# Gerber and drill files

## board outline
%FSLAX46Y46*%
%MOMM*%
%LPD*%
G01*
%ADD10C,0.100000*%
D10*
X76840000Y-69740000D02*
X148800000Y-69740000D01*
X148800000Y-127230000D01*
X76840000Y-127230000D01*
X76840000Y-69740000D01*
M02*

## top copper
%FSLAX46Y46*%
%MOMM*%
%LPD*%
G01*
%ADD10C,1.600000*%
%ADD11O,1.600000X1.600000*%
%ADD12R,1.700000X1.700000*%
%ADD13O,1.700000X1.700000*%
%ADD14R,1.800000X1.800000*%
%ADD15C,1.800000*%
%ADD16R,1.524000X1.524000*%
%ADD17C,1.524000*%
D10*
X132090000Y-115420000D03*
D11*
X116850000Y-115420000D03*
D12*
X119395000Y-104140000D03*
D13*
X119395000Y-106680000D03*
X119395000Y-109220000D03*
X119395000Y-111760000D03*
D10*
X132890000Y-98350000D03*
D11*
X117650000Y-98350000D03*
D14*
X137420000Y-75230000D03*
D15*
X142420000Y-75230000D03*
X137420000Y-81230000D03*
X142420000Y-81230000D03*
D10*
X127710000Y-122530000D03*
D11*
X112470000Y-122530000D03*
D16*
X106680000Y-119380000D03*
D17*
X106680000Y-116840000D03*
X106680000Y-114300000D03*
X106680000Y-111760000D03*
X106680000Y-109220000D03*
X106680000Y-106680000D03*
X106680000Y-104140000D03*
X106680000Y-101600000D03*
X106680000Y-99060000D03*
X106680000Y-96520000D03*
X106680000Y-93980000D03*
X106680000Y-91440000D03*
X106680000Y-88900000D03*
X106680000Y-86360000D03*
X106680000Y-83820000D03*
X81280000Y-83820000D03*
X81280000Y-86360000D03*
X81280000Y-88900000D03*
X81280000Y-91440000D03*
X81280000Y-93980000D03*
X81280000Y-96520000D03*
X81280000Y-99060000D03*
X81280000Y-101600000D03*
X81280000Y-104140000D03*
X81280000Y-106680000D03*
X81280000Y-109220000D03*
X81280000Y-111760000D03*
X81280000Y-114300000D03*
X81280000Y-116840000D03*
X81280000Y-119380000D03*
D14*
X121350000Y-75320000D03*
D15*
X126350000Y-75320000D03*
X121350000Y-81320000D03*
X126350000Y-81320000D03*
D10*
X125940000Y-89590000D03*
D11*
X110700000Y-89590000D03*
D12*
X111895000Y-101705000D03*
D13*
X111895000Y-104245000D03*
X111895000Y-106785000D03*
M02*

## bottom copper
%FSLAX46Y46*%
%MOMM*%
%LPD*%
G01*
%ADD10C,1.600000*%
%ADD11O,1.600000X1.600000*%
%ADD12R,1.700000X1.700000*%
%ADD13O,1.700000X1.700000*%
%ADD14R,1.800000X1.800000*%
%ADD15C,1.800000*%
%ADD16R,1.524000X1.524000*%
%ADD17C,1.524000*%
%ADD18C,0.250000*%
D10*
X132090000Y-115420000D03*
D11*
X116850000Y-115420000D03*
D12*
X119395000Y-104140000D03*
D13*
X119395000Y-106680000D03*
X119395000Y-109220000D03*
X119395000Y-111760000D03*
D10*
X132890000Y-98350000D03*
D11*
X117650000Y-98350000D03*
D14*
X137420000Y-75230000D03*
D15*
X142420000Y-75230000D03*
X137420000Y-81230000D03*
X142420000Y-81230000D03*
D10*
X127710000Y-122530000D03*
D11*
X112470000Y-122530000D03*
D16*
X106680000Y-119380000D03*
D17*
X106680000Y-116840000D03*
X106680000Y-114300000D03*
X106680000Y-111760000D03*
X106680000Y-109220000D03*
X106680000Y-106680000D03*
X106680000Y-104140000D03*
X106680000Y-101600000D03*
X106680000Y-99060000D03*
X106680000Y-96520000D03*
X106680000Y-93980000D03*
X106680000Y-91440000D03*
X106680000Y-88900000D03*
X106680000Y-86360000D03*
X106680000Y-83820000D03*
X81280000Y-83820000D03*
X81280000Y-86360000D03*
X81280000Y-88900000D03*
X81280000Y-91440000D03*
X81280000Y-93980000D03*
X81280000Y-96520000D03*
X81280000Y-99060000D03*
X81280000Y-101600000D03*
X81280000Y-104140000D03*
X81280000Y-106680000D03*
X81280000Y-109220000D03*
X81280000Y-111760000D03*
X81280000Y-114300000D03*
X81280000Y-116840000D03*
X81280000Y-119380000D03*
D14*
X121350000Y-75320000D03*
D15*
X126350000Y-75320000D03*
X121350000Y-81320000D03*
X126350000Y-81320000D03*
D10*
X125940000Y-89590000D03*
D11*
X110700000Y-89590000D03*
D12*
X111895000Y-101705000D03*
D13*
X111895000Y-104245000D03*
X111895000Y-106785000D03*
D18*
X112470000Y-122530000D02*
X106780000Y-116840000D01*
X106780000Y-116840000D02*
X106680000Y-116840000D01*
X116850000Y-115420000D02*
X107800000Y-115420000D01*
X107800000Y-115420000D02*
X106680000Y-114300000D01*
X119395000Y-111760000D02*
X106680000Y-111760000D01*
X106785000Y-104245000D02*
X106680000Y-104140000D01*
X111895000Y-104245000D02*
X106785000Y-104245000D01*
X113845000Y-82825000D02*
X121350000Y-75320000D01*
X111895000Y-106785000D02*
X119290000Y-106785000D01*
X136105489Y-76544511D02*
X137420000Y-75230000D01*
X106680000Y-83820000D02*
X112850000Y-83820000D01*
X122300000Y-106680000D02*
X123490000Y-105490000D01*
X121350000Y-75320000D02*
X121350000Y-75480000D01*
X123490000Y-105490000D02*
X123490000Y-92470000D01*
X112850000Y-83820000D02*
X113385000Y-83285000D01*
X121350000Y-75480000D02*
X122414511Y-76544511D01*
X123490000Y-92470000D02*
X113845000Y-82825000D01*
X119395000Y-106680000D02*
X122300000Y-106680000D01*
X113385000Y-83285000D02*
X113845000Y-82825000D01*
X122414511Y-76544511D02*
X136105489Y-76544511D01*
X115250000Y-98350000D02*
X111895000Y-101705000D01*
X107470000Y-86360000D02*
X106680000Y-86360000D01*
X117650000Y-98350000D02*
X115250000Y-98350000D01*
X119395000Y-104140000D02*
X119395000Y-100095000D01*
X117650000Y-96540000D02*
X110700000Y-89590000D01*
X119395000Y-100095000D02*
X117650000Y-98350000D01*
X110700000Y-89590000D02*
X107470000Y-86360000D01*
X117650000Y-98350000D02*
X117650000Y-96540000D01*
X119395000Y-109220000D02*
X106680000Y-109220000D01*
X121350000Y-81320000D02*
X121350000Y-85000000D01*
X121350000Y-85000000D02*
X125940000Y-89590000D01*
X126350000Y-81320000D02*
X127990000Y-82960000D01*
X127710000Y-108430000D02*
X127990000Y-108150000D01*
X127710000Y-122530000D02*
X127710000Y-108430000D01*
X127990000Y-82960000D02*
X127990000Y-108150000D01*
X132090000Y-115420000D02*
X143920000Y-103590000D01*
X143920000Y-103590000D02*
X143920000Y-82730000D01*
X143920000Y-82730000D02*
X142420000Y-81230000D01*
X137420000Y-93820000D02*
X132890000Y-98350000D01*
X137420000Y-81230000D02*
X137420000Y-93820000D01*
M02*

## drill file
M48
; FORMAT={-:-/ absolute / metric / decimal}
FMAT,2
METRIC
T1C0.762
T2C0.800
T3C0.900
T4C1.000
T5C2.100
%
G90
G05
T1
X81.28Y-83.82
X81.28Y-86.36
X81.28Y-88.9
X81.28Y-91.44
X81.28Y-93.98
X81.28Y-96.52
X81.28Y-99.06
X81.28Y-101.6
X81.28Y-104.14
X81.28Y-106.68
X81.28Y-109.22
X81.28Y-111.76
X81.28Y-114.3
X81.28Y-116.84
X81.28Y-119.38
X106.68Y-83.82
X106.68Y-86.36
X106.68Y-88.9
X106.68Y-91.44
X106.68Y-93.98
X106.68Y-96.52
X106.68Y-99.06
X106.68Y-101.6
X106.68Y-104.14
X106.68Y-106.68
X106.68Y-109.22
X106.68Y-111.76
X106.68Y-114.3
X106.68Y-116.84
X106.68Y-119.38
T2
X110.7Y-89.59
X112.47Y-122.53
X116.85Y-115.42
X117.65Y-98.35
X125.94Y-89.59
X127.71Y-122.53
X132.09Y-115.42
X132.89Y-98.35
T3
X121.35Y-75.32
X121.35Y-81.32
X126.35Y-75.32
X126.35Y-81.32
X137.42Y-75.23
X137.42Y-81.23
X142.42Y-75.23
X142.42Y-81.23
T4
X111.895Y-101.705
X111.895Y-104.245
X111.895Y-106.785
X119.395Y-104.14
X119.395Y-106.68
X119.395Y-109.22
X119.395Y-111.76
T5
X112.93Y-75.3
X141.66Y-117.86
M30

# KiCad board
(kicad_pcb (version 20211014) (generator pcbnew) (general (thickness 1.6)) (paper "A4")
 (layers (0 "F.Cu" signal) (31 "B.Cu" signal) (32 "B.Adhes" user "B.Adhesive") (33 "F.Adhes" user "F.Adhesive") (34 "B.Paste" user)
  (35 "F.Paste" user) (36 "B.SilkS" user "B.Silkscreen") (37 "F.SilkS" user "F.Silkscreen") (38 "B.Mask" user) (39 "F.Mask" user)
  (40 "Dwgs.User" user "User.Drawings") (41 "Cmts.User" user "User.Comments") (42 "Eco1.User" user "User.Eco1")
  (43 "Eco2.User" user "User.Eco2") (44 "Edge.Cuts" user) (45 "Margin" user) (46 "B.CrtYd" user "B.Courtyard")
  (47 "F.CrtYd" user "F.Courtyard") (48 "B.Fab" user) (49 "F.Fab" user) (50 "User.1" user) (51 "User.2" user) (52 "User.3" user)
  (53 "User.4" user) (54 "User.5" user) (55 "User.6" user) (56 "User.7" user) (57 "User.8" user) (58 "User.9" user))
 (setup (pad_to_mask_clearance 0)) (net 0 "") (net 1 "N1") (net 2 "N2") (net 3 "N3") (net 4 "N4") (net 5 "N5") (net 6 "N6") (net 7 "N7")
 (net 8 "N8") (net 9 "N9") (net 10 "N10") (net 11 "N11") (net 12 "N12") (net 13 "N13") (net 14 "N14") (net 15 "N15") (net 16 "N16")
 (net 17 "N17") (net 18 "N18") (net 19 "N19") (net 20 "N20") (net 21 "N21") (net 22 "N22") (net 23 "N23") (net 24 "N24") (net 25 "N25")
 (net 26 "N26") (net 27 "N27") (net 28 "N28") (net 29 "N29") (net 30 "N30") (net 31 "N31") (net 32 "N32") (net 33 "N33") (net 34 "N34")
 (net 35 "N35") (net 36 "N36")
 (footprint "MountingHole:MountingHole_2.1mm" (layer "F.Cu") (at 112.93 75.3)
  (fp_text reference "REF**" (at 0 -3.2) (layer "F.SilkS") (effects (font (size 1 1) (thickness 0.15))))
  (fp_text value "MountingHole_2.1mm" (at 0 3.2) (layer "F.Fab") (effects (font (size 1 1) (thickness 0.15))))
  (pad "" np_thru_hole circle (at 0 0) (size 2.1 2.1) (drill 2.1) (layers *.Cu *.Mask)))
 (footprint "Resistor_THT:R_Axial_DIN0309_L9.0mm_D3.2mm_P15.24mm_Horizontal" (layer "F.Cu") (at 132.09 115.42 180)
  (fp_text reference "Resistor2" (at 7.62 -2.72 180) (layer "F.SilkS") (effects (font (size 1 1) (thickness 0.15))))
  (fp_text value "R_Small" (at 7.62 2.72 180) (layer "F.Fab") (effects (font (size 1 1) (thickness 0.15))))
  (pad "1" thru_hole circle (at 0 0 180) (size 1.6 1.6) (drill 0.8) (layers *.Cu *.Mask) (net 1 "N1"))
  (pad "2" thru_hole oval (at 15.24 0 180) (size 1.6 1.6) (drill 0.8) (layers *.Cu *.Mask) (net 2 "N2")))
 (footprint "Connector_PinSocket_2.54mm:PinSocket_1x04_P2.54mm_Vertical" (layer "F.Cu") (at 119.395 104.14)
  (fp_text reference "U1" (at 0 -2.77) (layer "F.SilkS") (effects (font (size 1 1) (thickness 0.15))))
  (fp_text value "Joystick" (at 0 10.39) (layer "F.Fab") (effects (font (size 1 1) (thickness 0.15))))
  (pad "1" thru_hole rect (at 0 0) (size 1.7 1.7) (drill 1) (layers *.Cu *.Mask) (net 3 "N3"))
  (pad "2" thru_hole oval (at 0 2.54) (size 1.7 1.7) (drill 1) (layers *.Cu *.Mask) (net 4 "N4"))
  (pad "3" thru_hole oval (at 0 5.08) (size 1.7 1.7) (drill 1) (layers *.Cu *.Mask) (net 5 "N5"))
  (pad "4" thru_hole oval (at 0 7.62) (size 1.7 1.7) (drill 1) (layers *.Cu *.Mask) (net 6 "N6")))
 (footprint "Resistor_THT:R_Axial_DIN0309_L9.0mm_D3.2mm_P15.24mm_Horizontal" (layer "F.Cu") (at 132.89 98.35 180)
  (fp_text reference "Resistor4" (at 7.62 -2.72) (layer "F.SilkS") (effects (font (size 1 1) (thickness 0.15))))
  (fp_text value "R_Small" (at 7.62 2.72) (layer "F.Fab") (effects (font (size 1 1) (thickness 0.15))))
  (pad "1" thru_hole circle (at 0 0 180) (size 1.6 1.6) (drill 0.8) (layers *.Cu *.Mask) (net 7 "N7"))
  (pad "2" thru_hole oval (at 15.24 0 180) (size 1.6 1.6) (drill 0.8) (layers *.Cu *.Mask) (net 3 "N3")))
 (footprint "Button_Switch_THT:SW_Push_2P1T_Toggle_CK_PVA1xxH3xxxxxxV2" (layer "F.Cu") (at 137.42 75.23)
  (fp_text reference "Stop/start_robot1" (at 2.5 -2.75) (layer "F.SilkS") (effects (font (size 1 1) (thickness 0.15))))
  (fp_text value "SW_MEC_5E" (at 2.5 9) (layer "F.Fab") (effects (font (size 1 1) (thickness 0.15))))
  (pad "1" thru_hole rect (at 0 0) (size 1.8 1.8) (drill 0.9) (layers *.Cu *.Mask) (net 4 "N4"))
  (pad "2" thru_hole circle (at 5 0) (size 1.8 1.8) (drill 0.9) (layers *.Cu *.Mask) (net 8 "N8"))
  (pad "3" thru_hole circle (at 0 6) (size 1.8 1.8) (drill 0.9) (layers *.Cu *.Mask) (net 7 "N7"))
  (pad "4" thru_hole circle (at 5 6) (size 1.8 1.8) (drill 0.9) (layers *.Cu *.Mask) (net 1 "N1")))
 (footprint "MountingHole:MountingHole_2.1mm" (layer "F.Cu") (at 141.66 117.86)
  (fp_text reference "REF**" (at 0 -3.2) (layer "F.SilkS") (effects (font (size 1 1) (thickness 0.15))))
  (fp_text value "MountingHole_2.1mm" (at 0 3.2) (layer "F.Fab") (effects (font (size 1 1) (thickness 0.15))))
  (pad "" np_thru_hole circle (at 0 0) (size 2.1 2.1) (drill 2.1) (layers *.Cu *.Mask)))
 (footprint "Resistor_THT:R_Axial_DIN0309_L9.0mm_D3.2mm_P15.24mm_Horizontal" (layer "F.Cu") (at 127.71 122.53 180)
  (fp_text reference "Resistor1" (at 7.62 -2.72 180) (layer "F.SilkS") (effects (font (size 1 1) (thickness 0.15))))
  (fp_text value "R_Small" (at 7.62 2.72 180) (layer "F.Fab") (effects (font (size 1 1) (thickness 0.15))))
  (pad "1" thru_hole circle (at 0 0 180) (size 1.6 1.6) (drill 0.8) (layers *.Cu *.Mask) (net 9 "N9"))
  (pad "2" thru_hole oval (at 15.24 0 180) (size 1.6 1.6) (drill 0.8) (layers *.Cu *.Mask) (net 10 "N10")))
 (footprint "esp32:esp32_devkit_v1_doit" (layer "F.Cu") (at 93.98 119.38 180)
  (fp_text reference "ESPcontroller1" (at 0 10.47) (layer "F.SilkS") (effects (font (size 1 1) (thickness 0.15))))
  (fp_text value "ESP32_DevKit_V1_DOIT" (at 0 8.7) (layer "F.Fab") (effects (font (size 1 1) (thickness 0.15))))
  (pad "1" thru_hole rect locked (at -12.7 0 180) (size 1.524 1.524) (drill 0.762) (layers *.Cu *.Mask) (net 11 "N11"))
  (pad "2" thru_hole circle locked (at -12.7 2.54 180) (size 1.524 1.524) (drill 0.762) (layers *.Cu *.Mask) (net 10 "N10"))
  (pad "3" thru_hole circle locked (at -12.7 5.08 180) (size 1.524 1.524) (drill 0.762) (layers *.Cu *.Mask) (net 2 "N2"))
  (pad "4" thru_hole circle locked (at -12.7 7.62 180) (size 1.524 1.524) (drill 0.762) (layers *.Cu *.Mask) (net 6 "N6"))
  (pad "5" thru_hole circle locked (at -12.7 10.16 180) (size 1.524 1.524) (drill 0.762) (layers *.Cu *.Mask) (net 5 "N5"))
  (pad "6" thru_hole circle locked (at -12.7 12.7 180) (size 1.524 1.524) (drill 0.762) (layers *.Cu *.Mask) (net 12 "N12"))
  (pad "7" thru_hole circle locked (at -12.7 15.24 180) (size 1.524 1.524) (drill 0.762) (layers *.Cu *.Mask) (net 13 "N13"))
  (pad "8" thru_hole circle locked (at -12.7 17.78 180) (size 1.524 1.524) (drill 0.762) (layers *.Cu *.Mask) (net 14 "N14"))
  (pad "9" thru_hole circle locked (at -12.7 20.32 180) (size 1.524 1.524) (drill 0.762) (layers *.Cu *.Mask) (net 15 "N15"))
  (pad "10" thru_hole circle locked (at -12.7 22.86 180) (size 1.524 1.524) (drill 0.762) (layers *.Cu *.Mask) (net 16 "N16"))
  (pad "11" thru_hole circle locked (at -12.7 25.4 180) (size 1.524 1.524) (drill 0.762) (layers *.Cu *.Mask) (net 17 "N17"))
  (pad "12" thru_hole circle locked (at -12.7 27.94 180) (size 1.524 1.524) (drill 0.762) (layers *.Cu *.Mask) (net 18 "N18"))
  (pad "13" thru_hole circle locked (at -12.7 30.48 180) (size 1.524 1.524) (drill 0.762) (layers *.Cu *.Mask) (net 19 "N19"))
  (pad "14" thru_hole circle locked (at -12.7 33.02 180) (size 1.524 1.524) (drill 0.762) (layers *.Cu *.Mask) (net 3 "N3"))
  (pad "15" thru_hole circle locked (at -12.7 35.56 180) (size 1.524 1.524) (drill 0.762) (layers *.Cu *.Mask) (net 4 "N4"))
  (pad "16" thru_hole circle locked (at 12.7 35.56 180) (size 1.524 1.524) (drill 0.762) (layers *.Cu *.Mask) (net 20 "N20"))
  (pad "17" thru_hole circle locked (at 12.7 33.02 180) (size 1.524 1.524) (drill 0.762) (layers *.Cu *.Mask) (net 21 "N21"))
  (pad "18" thru_hole circle locked (at 12.7 30.48 180) (size 1.524 1.524) (drill 0.762) (layers *.Cu *.Mask) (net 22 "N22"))
  (pad "19" thru_hole circle locked (at 12.7 27.94 180) (size 1.524 1.524) (drill 0.762) (layers *.Cu *.Mask) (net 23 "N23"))
  (pad "20" thru_hole circle locked (at 12.7 25.4 180) (size 1.524 1.524) (drill 0.762) (layers *.Cu *.Mask) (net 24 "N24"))
  (pad "21" thru_hole circle locked (at 12.7 22.86 180) (size 1.524 1.524) (drill 0.762) (layers *.Cu *.Mask) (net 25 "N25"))
  (pad "22" thru_hole circle locked (at 12.7 20.32 180) (size 1.524 1.524) (drill 0.762) (layers *.Cu *.Mask) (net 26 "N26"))
  (pad "23" thru_hole circle locked (at 12.7 17.78 180) (size 1.524 1.524) (drill 0.762) (layers *.Cu *.Mask) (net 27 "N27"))
  (pad "24" thru_hole circle locked (at 12.7 15.24 180) (size 1.524 1.524) (drill 0.762) (layers *.Cu *.Mask) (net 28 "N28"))
  (pad "25" thru_hole circle locked (at 12.7 12.7 180) (size 1.524 1.524) (drill 0.762) (layers *.Cu *.Mask) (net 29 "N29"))
  (pad "26" thru_hole circle locked (at 12.7 10.16 180) (size 1.524 1.524) (drill 0.762) (layers *.Cu *.Mask) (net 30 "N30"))
  (pad "27" thru_hole circle locked (at 12.7 7.62 180) (size 1.524 1.524) (drill 0.762) (layers *.Cu *.Mask) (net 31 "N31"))
  (pad "28" thru_hole circle locked (at 12.7 5.08 180) (size 1.524 1.524) (drill 0.762) (layers *.Cu *.Mask) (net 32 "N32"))
  (pad "29" thru_hole circle locked (at 12.7 2.54 180) (size 1.524 1.524) (drill 0.762) (layers *.Cu *.Mask) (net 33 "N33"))
  (pad "30" thru_hole circle locked (at 12.7 0 180) (size 1.524 1.524) (drill 0.762) (layers *.Cu *.Mask) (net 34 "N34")))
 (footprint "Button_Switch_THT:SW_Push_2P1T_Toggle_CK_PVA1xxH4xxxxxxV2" (layer "F.Cu") (at 121.35 75.32)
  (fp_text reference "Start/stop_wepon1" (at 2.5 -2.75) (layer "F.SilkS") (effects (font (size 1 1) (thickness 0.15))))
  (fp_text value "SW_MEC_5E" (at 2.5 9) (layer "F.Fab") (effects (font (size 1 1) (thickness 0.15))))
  (pad "1" thru_hole rect (at 0 0) (size 1.8 1.8) (drill 0.9) (layers *.Cu *.Mask) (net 4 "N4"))
  (pad "2" thru_hole circle (at 5 0) (size 1.8 1.8) (drill 0.9) (layers *.Cu *.Mask) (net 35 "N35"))
  (pad "3" thru_hole circle (at 0 6) (size 1.8 1.8) (drill 0.9) (layers *.Cu *.Mask) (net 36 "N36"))
  (pad "4" thru_hole circle (at 5 6) (size 1.8 1.8) (drill 0.9) (layers *.Cu *.Mask) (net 9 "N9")))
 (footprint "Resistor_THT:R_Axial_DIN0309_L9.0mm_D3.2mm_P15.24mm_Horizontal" (layer "F.Cu") (at 125.94 89.59 180)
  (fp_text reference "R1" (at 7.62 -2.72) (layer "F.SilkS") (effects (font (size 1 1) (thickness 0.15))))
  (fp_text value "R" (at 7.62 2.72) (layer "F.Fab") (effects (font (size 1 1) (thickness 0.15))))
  (pad "1" thru_hole circle (at 0 0 180) (size 1.6 1.6) (drill 0.8) (layers *.Cu *.Mask) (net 36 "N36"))
  (pad "2" thru_hole oval (at 15.24 0 180) (size 1.6 1.6) (drill 0.8) (layers *.Cu *.Mask) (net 3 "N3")))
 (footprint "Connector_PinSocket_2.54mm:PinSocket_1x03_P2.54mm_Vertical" (layer "F.Cu") (at 111.895 101.705)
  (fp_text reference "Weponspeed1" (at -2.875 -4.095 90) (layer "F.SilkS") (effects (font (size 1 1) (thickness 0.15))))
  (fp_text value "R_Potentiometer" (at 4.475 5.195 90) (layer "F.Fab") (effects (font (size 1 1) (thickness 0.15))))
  (pad "1" thru_hole rect (at 0 0) (size 1.7 1.7) (drill 1) (layers *.Cu *.Mask) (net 3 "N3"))
  (pad "2" thru_hole oval (at 0 2.54) (size 1.7 1.7) (drill 1) (layers *.Cu *.Mask) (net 13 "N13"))
  (pad "3" thru_hole oval (at 0 5.08) (size 1.7 1.7) (drill 1) (layers *.Cu *.Mask) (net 4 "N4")))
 (gr_rect (start 76.84 69.74) (end 148.8 127.23) (layer "Edge.Cuts") (width 0.1) (fill none))
 (segment (start 112.47 122.53) (end 106.78 116.84) (width 0.25) (layer "B.Cu") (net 10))
 (segment (start 106.78 116.84) (end 106.68 116.84) (width 0.25) (layer "B.Cu") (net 10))
 (segment (start 116.85 115.42) (end 107.8 115.42) (width 0.25) (layer "B.Cu") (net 2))
 (segment (start 107.8 115.42) (end 106.68 114.3) (width 0.25) (layer "B.Cu") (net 2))
 (segment (start 119.395 111.76) (end 106.68 111.76) (width 0.25) (layer "B.Cu") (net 6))
 (segment (start 106.785 104.245) (end 106.68 104.14) (width 0.25) (layer "B.Cu") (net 13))
 (segment (start 111.895 104.245) (end 106.785 104.245) (width 0.25) (layer "B.Cu") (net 13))
 (segment (start 113.845 82.825) (end 121.35 75.32) (width 0.25) (layer "B.Cu") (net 4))
 (segment (start 111.895 106.785) (end 119.29 106.785) (width 0.25) (layer "B.Cu") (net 4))
 (segment (start 136.105489 76.544511) (end 137.42 75.23) (width 0.25) (layer "B.Cu") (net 4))
 (segment (start 106.68 83.82) (end 112.85 83.82) (width 0.25) (layer "B.Cu") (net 4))
 (segment (start 122.3 106.68) (end 123.49 105.49) (width 0.25) (layer "B.Cu") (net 4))
 (segment (start 121.35 75.32) (end 121.35 75.48) (width 0.25) (layer "B.Cu") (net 4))
 (segment (start 123.49 105.49) (end 123.49 92.47) (width 0.25) (layer "B.Cu") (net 4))
 (segment (start 112.85 83.82) (end 113.385 83.285) (width 0.25) (layer "B.Cu") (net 4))
 (segment (start 121.35 75.48) (end 122.414511 76.544511) (width 0.25) (layer "B.Cu") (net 4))
 (segment (start 123.49 92.47) (end 113.845 82.825) (width 0.25) (layer "B.Cu") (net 4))
 (segment (start 119.395 106.68) (end 122.3 106.68) (width 0.25) (layer "B.Cu") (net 4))
 (segment (start 113.385 83.285) (end 113.845 82.825) (width 0.25) (layer "B.Cu") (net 4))
 (segment (start 122.414511 76.544511) (end 136.105489 76.544511) (width 0.25) (layer "B.Cu") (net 4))
 (segment (start 115.25 98.35) (end 111.895 101.705) (width 0.25) (layer "B.Cu") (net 3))
 (segment (start 107.47 86.36) (end 106.68 86.36) (width 0.25) (layer "B.Cu") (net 3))
 (segment (start 117.65 98.35) (end 115.25 98.35) (width 0.25) (layer "B.Cu") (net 3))
 (segment (start 119.395 104.14) (end 119.395 100.095) (width 0.25) (layer "B.Cu") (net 3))
 (segment (start 117.65 96.54) (end 110.7 89.59) (width 0.25) (layer "B.Cu") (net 3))
 (segment (start 119.395 100.095) (end 117.65 98.35) (width 0.25) (layer "B.Cu") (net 3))
 (segment (start 110.7 89.59) (end 107.47 86.36) (width 0.25) (layer "B.Cu") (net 3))
 (segment (start 117.65 98.35) (end 117.65 96.54) (width 0.25) (layer "B.Cu") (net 3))
 (segment (start 119.395 109.22) (end 106.68 109.22) (width 0.25) (layer "B.Cu") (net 5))
 (segment (start 121.35 81.32) (end 121.35 85) (width 0.25) (layer "B.Cu") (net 36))
 (segment (start 121.35 85) (end 125.94 89.59) (width 0.25) (layer "B.Cu") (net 36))
 (segment (start 126.35 81.32) (end 127.99 82.96) (width 0.25) (layer "B.Cu") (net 9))
 (segment (start 127.71 108.43) (end 127.99 108.15) (width 0.25) (layer "B.Cu") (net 9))
 (segment (start 127.71 122.53) (end 127.71 108.43) (width 0.25) (layer "B.Cu") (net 9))
 (segment (start 127.99 82.96) (end 127.99 108.15) (width 0.25) (layer "B.Cu") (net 9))
 (segment (start 132.09 115.42) (end 143.92 103.59) (width 0.25) (layer "B.Cu") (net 1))
 (segment (start 143.92 103.59) (end 143.92 82.73) (width 0.25) (layer "B.Cu") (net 1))
 (segment (start 143.92 82.73) (end 142.42 81.23) (width 0.25) (layer "B.Cu") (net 1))
 (segment (start 137.42 93.82) (end 132.89 98.35) (width 0.25) (layer "B.Cu") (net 7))
 (segment (start 137.42 81.23) (end 137.42 93.82) (width 0.25) (layer "B.Cu") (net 7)))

